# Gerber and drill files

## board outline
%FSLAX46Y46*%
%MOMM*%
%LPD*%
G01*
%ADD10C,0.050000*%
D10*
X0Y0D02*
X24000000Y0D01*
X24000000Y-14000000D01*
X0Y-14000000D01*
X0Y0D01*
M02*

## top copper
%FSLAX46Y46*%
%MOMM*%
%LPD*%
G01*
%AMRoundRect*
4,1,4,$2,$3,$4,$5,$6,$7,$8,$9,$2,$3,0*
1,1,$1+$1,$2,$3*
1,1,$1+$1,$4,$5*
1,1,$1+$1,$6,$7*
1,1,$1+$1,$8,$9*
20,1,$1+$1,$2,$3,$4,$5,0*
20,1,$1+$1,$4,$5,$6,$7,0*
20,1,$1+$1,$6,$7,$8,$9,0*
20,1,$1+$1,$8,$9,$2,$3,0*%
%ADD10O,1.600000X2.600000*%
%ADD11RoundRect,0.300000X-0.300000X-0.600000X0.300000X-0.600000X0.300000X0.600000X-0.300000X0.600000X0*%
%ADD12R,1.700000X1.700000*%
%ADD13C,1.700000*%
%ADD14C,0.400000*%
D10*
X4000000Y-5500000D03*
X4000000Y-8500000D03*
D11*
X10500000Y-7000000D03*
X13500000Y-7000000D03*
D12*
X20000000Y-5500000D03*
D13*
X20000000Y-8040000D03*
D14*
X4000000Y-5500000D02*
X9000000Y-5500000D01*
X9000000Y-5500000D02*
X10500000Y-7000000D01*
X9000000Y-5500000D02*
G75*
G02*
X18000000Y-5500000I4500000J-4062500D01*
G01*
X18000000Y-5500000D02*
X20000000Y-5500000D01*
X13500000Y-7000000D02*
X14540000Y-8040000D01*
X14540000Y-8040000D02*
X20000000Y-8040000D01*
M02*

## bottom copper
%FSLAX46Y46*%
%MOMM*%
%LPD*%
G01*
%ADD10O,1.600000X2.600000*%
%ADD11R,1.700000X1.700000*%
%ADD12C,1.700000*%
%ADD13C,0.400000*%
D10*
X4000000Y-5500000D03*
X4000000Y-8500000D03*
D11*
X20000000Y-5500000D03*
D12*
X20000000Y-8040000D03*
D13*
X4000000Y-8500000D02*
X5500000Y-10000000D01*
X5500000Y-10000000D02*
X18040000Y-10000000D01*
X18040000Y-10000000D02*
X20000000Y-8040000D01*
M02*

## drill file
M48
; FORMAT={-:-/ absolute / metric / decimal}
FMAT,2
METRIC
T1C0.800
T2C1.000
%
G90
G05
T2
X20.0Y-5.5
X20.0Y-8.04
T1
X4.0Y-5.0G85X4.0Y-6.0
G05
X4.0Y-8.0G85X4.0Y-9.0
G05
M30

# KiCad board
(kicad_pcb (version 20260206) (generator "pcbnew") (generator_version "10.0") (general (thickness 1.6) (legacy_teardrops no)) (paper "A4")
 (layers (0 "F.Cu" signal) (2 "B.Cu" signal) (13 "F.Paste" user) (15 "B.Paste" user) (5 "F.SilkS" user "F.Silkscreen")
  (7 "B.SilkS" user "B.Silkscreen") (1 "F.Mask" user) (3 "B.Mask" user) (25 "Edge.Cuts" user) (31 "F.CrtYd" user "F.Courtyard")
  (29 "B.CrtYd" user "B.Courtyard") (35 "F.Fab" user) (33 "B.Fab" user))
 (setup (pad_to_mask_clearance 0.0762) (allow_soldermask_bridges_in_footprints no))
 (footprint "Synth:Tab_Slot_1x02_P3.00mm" (layer "F.Cu") (at 4 7)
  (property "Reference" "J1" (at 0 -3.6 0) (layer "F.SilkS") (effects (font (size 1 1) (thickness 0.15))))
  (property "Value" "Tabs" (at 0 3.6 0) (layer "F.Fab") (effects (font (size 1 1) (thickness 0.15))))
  (pad "1" thru_hole oval (at 0 -1.5) (size 1.6 2.6) (drill oval 0.8 1.8) (layers "*.Cu" "*.Mask") (remove_unused_layers no) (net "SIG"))
  (pad "2" thru_hole oval (at 0 1.5) (size 1.6 2.6) (drill oval 0.8 1.8) (layers "*.Cu" "*.Mask") (remove_unused_layers no) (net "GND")))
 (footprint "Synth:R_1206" (layer "F.Cu") (at 12 7)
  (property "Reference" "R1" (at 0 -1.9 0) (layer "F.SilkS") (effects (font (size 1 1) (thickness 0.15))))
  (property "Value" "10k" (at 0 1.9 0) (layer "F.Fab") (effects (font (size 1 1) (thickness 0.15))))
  (pad "1" smd roundrect (at -1.5 0) (size 1.2 1.8) (layers "F.Cu" "F.Paste" "F.Mask") (roundrect_rratio 0.25) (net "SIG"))
  (pad "2" smd roundrect (at 1.5 0) (size 1.2 1.8) (layers "F.Cu" "F.Paste" "F.Mask") (roundrect_rratio 0.25) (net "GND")))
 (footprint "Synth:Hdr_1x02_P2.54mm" (layer "B.Cu") (at 20 6.77)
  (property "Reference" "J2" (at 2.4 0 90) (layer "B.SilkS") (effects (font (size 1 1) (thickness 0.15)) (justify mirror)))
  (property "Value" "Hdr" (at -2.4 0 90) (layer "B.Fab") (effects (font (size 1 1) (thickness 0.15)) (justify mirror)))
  (pad "1" thru_hole rect (at 0 -1.27) (size 1.7 1.7) (drill 1) (layers "*.Cu" "*.Mask") (remove_unused_layers no) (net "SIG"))
  (pad "2" thru_hole circle (at 0 1.27) (size 1.7 1.7) (drill 1) (layers "*.Cu" "*.Mask") (remove_unused_layers no) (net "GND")))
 (gr_rect (start 0 0) (end 24 14) (stroke (width 0.05) (type default)) (fill no) (layer "Edge.Cuts"))
 (segment (start 4 5.5) (end 9 5.5) (width 0.4) (layer "F.Cu") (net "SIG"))
 (segment (start 9 5.5) (end 10.5 7) (width 0.4) (layer "F.Cu") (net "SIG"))
 (arc (start 9 5.5) (mid 13.5 3.5) (end 18 5.5) (width 0.4) (layer "F.Cu") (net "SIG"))
 (segment (start 18 5.5) (end 20 5.5) (width 0.4) (layer "F.Cu") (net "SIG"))
 (segment (start 13.5 7) (end 14.54 8.04) (width 0.4) (layer "F.Cu") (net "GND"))
 (segment (start 14.54 8.04) (end 20 8.04) (width 0.4) (layer "F.Cu") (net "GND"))
 (segment (start 4 8.5) (end 5.5 10) (width 0.4) (layer "B.Cu") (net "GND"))
 (segment (start 5.5 10) (end 18.04 10) (width 0.4) (layer "B.Cu") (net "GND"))
 (segment (start 18.04 10) (end 20 8.04) (width 0.4) (layer "B.Cu") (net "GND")))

